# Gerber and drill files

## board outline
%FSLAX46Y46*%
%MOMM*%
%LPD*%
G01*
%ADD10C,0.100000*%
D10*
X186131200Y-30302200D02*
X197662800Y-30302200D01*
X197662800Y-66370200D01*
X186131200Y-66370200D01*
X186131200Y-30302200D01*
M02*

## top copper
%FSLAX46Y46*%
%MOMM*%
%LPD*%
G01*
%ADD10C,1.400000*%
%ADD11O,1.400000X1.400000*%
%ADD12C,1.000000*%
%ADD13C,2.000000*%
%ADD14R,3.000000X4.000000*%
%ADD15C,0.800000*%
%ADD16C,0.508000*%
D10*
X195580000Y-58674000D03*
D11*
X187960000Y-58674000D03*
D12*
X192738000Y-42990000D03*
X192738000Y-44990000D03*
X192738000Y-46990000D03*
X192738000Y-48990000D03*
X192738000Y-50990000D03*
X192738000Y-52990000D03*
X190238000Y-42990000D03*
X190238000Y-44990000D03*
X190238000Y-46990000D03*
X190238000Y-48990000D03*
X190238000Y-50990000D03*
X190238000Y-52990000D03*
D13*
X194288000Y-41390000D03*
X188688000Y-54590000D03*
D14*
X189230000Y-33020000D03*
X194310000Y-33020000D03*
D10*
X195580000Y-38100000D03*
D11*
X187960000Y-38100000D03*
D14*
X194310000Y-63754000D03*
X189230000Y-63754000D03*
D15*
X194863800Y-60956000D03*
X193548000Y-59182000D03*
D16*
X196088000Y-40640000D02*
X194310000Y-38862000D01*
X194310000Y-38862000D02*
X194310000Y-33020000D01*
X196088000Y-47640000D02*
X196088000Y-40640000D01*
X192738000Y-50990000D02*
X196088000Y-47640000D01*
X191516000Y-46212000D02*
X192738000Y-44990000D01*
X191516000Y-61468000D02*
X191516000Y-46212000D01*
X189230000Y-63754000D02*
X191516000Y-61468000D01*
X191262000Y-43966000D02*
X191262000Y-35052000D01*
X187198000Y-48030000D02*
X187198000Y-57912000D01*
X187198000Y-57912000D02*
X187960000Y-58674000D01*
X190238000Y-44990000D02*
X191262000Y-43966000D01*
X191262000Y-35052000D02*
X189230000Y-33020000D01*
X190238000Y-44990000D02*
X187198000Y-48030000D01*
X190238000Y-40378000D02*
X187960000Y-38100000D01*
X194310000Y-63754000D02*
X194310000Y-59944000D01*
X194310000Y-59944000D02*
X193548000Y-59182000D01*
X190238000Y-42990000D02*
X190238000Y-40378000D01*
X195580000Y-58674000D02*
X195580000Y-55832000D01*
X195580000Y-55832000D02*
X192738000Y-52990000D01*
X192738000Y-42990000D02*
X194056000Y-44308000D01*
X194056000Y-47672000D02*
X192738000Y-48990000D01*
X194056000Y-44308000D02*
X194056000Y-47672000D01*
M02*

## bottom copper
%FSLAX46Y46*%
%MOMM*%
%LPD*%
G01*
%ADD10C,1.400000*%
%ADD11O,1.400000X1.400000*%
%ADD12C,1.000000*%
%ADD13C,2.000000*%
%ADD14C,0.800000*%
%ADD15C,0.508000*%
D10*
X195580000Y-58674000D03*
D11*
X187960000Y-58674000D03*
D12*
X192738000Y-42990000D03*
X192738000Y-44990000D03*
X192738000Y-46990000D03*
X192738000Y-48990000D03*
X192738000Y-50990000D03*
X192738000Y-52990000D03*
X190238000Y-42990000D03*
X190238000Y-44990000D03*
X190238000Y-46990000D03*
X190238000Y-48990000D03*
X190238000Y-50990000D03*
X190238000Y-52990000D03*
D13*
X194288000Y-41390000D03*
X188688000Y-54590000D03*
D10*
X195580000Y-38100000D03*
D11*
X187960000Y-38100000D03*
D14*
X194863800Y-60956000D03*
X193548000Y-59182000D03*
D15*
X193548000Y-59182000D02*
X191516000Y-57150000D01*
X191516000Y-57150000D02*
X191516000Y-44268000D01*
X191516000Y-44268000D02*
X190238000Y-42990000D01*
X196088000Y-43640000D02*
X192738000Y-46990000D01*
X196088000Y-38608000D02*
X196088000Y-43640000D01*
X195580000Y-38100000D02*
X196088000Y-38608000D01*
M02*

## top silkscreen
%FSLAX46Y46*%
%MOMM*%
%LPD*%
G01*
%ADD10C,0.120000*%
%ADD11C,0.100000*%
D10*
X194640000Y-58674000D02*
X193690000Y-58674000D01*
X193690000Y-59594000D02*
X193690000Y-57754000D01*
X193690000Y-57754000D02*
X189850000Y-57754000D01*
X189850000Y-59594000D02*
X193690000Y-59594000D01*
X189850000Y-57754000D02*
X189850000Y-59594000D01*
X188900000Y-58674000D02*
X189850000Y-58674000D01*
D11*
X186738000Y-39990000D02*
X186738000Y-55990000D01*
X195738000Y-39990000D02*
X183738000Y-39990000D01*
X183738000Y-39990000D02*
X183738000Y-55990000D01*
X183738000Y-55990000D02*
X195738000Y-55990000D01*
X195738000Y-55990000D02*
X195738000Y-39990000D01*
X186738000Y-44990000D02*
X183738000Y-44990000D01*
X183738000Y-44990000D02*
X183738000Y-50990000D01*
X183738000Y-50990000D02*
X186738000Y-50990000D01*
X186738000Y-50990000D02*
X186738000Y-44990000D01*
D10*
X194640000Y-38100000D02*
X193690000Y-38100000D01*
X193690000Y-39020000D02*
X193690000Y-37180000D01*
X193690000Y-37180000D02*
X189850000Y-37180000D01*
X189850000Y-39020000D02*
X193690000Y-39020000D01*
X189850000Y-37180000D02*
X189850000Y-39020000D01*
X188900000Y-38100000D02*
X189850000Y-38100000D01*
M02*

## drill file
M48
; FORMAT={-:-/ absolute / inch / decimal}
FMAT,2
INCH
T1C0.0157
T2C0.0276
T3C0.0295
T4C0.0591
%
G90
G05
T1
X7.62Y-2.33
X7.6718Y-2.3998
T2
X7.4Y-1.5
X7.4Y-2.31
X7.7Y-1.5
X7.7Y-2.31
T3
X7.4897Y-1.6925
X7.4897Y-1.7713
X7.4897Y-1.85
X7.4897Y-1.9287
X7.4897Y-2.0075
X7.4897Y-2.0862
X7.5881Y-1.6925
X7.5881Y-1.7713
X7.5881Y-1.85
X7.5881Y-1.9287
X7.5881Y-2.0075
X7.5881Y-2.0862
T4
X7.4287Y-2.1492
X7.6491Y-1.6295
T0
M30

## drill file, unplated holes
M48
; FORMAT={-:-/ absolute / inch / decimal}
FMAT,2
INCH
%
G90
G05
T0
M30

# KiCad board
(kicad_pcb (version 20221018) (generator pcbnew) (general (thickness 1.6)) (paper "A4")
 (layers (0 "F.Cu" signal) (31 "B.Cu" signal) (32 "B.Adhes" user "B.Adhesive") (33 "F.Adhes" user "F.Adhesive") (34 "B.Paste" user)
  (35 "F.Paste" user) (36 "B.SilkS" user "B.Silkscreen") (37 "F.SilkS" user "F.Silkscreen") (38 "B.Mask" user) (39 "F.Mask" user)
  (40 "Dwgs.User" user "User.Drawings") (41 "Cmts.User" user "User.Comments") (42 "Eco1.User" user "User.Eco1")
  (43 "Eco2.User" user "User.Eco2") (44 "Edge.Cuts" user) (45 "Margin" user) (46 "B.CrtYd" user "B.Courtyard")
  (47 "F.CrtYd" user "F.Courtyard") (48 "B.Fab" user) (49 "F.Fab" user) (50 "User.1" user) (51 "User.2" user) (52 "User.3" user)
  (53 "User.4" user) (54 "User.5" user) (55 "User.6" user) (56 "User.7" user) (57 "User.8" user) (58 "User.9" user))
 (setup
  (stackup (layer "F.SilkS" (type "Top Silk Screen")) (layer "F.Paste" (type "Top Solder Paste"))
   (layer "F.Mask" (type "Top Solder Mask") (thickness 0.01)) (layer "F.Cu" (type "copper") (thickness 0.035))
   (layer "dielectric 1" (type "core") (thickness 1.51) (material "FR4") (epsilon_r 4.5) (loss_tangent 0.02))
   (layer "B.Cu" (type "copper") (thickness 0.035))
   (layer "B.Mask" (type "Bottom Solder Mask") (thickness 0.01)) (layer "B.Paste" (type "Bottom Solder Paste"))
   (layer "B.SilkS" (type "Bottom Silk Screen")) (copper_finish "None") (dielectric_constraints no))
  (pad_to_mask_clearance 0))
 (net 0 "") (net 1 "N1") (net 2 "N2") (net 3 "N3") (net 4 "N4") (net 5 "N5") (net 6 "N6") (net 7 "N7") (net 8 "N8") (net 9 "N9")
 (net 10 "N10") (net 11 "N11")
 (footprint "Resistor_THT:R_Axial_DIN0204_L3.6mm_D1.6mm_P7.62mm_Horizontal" (layer "F.Cu") (at 195.58 58.674 180)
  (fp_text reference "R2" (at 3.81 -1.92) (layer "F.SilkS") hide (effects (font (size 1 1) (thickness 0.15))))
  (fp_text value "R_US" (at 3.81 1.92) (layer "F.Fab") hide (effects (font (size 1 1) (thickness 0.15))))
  (fp_line (start 0.94 0) (end 1.89 0) (stroke (width 0.12) (type solid)) (layer "F.SilkS"))
  (fp_line (start 1.89 -0.92) (end 1.89 0.92) (stroke (width 0.12) (type solid)) (layer "F.SilkS"))
  (fp_line (start 1.89 0.92) (end 5.73 0.92) (stroke (width 0.12) (type solid)) (layer "F.SilkS"))
  (fp_line (start 5.73 -0.92) (end 1.89 -0.92) (stroke (width 0.12) (type solid)) (layer "F.SilkS"))
  (fp_line (start 5.73 0.92) (end 5.73 -0.92) (stroke (width 0.12) (type solid)) (layer "F.SilkS"))
  (fp_line (start 6.68 0) (end 5.73 0) (stroke (width 0.12) (type solid)) (layer "F.SilkS"))
  (pad "1" thru_hole circle (at 0 0 180) (size 1.4 1.4) (drill 0.7) (layers "*.Cu" "*.Mask") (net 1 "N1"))
  (pad "2" thru_hole oval (at 7.62 0 180) (size 1.4 1.4) (drill 0.7) (layers "*.Cu" "*.Mask") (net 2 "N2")))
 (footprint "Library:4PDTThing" (layer "F.Cu") (at 185.738 46.99 -90)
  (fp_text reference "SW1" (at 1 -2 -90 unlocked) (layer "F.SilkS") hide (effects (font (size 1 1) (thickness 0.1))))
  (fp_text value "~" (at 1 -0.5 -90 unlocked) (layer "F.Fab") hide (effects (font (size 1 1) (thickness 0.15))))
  (fp_line (start -7 -1) (end 9 -1) (stroke (width 0.1) (type default)) (layer "F.SilkS"))
  (fp_rect (start -7 -10) (end 9 2) (stroke (width 0.1) (type default)) (fill none) (layer "F.SilkS"))
  (fp_rect (start -2 -1) (end 4 2) (stroke (width 0.1) (type default)) (fill none) (layer "F.SilkS"))
  (pad "1" thru_hole circle (at -4 -7 270) (size 1 1) (drill 0.75) (layers "*.Cu" "*.Mask") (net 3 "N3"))
  (pad "2" thru_hole circle (at -2 -7 270) (size 1 1) (drill 0.75) (layers "*.Cu" "*.Mask") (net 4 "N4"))
  (pad "3" thru_hole circle (at 0 -7 270) (size 1 1) (drill 0.75) (layers "*.Cu" "*.Mask") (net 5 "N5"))
  (pad "4" thru_hole circle (at 2 -7 270) (size 1 1) (drill 0.75) (layers "*.Cu" "*.Mask") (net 3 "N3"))
  (pad "5" thru_hole circle (at 4 -7 270) (size 1 1) (drill 0.75) (layers "*.Cu" "*.Mask") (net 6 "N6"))
  (pad "6" thru_hole circle (at 6 -7 270) (size 1 1) (drill 0.75) (layers "*.Cu" "*.Mask") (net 1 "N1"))
  (pad "7" thru_hole circle (at -4 -4.5 270) (size 1 1) (drill 0.75) (layers "*.Cu" "*.Mask") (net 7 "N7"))
  (pad "8" thru_hole circle (at -2 -4.5 270) (size 1 1) (drill 0.75) (layers "*.Cu" "*.Mask") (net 2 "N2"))
  (pad "9" thru_hole circle (at 0 -4.5 270) (size 1 1) (drill 0.75) (layers "*.Cu" "*.Mask") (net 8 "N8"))
  (pad "10" thru_hole circle (at 2 -4.5 270) (size 1 1) (drill 0.75) (layers "*.Cu" "*.Mask") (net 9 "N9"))
  (pad "11" thru_hole circle (at 4 -4.5 270) (size 1 1) (drill 0.75) (layers "*.Cu" "*.Mask") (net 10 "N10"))
  (pad "12" thru_hole circle (at 6 -4.5 270) (size 1 1) (drill 0.75) (layers "*.Cu" "*.Mask") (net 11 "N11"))
  (pad "13" thru_hole circle (at -5.6 -8.55 270) (size 2 2) (drill 1.5) (layers "*.Cu" "*.Mask"))
  (pad "14" thru_hole circle (at 7.6 -2.95 270) (size 2 2) (drill 1.5) (layers "*.Cu" "*.Mask")))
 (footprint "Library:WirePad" (layer "F.Cu") (at 191.77 38.1)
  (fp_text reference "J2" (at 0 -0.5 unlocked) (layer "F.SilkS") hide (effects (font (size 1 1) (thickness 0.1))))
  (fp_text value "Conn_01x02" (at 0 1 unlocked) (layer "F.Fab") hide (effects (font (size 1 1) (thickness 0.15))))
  (pad "1" smd rect (at -2.54 -5.08 90) (size 4 3) (layers "F.Cu" "F.Paste" "F.Mask") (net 2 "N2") (thermal_bridge_angle 45))
  (pad "2" smd rect (at 2.54 -5.08 90) (size 4 3) (layers "F.Cu" "F.Paste" "F.Mask") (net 6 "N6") (thermal_bridge_angle 45)))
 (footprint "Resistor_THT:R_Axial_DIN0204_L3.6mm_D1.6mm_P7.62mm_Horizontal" (layer "F.Cu") (at 195.58 38.1 180)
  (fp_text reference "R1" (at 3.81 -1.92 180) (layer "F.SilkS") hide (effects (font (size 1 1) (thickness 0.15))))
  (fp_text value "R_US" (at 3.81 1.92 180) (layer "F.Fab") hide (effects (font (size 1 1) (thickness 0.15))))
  (fp_line (start 0.94 0) (end 1.89 0) (stroke (width 0.12) (type solid)) (layer "F.SilkS"))
  (fp_line (start 1.89 -0.92) (end 1.89 0.92) (stroke (width 0.12) (type solid)) (layer "F.SilkS"))
  (fp_line (start 1.89 0.92) (end 5.73 0.92) (stroke (width 0.12) (type solid)) (layer "F.SilkS"))
  (fp_line (start 5.73 -0.92) (end 1.89 -0.92) (stroke (width 0.12) (type solid)) (layer "F.SilkS"))
  (fp_line (start 5.73 0.92) (end 5.73 -0.92) (stroke (width 0.12) (type solid)) (layer "F.SilkS"))
  (fp_line (start 6.68 0) (end 5.73 0) (stroke (width 0.12) (type solid)) (layer "F.SilkS"))
  (pad "1" thru_hole circle (at 0 0 180) (size 1.4 1.4) (drill 0.7) (layers "*.Cu" "*.Mask") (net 5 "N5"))
  (pad "2" thru_hole oval (at 7.62 0 180) (size 1.4 1.4) (drill 0.7) (layers "*.Cu" "*.Mask") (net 7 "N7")))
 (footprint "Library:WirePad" (layer "F.Cu") (at 191.77 58.674 180)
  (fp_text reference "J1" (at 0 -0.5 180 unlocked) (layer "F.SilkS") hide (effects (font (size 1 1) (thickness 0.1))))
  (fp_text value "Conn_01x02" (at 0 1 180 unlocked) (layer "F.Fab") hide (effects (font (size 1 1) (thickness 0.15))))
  (pad "1" smd rect (at -2.54 -5.08 270) (size 4 3) (layers "F.Cu" "F.Paste" "F.Mask") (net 7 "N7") (thermal_bridge_angle 45))
  (pad "2" smd rect (at 2.54 -5.08 270) (size 4 3) (layers "F.Cu" "F.Paste" "F.Mask") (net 4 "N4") (thermal_bridge_angle 45)))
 (gr_rect (start 186.1312 30.3022) (end 197.6628 66.3702) (stroke (width 0.1) (type default)) (fill none) (layer "Edge.Cuts"))
 (segment (start 191.262 43.966) (end 191.262 35.052) (width 0.508) (layer "F.Cu") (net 2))
 (segment (start 187.198 48.03) (end 187.198 57.912) (width 0.508) (layer "F.Cu") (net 2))
 (segment (start 187.198 57.912) (end 187.96 58.674) (width 0.508) (layer "F.Cu") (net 2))
 (segment (start 190.238 44.99) (end 191.262 43.966) (width 0.508) (layer "F.Cu") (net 2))
 (segment (start 191.262 35.052) (end 189.23 33.02) (width 0.508) (layer "F.Cu") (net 2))
 (segment (start 190.238 44.99) (end 187.198 48.03) (width 0.508) (layer "F.Cu") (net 2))
 (segment (start 194.31 38.862) (end 194.31 33.02) (width 0.508) (layer "F.Cu") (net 6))
 (segment (start 196.088 47.64) (end 196.088 40.64) (width 0.508) (layer "F.Cu") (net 6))
 (segment (start 196.088 40.64) (end 194.31 38.862) (width 0.508) (layer "F.Cu") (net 6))
 (segment (start 192.738 50.99) (end 196.088 47.64) (width 0.508) (layer "F.Cu") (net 6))
 (segment (start 190.238 40.378) (end 187.96 38.1) (width 0.508) (layer "F.Cu") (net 7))
 (segment (start 194.31 63.754) (end 194.31 59.944) (width 0.508) (layer "F.Cu") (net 7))
 (segment (start 194.31 59.944) (end 193.548 59.182) (width 0.508) (layer "F.Cu") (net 7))
 (segment (start 190.238 42.99) (end 190.238 40.378) (width 0.508) (layer "F.Cu") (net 7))
 (via (at 194.8638 60.956) (size 0.8) (drill 0.4) (layers "F.Cu" "B.Cu") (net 7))
 (via (at 193.548 59.182) (size 0.8) (drill 0.4) (layers "F.Cu" "B.Cu") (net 7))
 (segment (start 193.548 59.182) (end 191.516 57.15) (width 0.508) (layer "B.Cu") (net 7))
 (segment (start 191.516 57.15) (end 191.516 44.268) (width 0.508) (layer "B.Cu") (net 7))
 (segment (start 191.516 44.268) (end 190.238 42.99) (width 0.508) (layer "B.Cu") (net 7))
 (segment (start 191.516 61.468) (end 191.516 46.212) (width 0.508) (layer "F.Cu") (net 4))
 (segment (start 189.23 63.754) (end 191.516 61.468) (width 0.508) (layer "F.Cu") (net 4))
 (segment (start 191.516 46.212) (end 192.738 44.99) (width 0.508) (layer "F.Cu") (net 4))
 (segment (start 196.088 43.64) (end 192.738 46.99) (width 0.508) (layer "B.Cu") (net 5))
 (segment (start 196.088 38.608) (end 196.088 43.64) (width 0.508) (layer "B.Cu") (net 5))
 (segment (start 195.58 38.1) (end 196.088 38.608) (width 0.508) (layer "B.Cu") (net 5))
 (segment (start 195.58 58.674) (end 195.58 55.832) (width 0.508) (layer "F.Cu") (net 1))
 (segment (start 195.58 55.832) (end 192.738 52.99) (width 0.508) (layer "F.Cu") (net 1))
 (segment (start 192.738 42.99) (end 194.056 44.308) (width 0.508) (layer "F.Cu") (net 3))
 (segment (start 194.056 47.672) (end 192.738 48.99) (width 0.508) (layer "F.Cu") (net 3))
 (segment (start 194.056 44.308) (end 194.056 47.672) (width 0.508) (layer "F.Cu") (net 3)))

